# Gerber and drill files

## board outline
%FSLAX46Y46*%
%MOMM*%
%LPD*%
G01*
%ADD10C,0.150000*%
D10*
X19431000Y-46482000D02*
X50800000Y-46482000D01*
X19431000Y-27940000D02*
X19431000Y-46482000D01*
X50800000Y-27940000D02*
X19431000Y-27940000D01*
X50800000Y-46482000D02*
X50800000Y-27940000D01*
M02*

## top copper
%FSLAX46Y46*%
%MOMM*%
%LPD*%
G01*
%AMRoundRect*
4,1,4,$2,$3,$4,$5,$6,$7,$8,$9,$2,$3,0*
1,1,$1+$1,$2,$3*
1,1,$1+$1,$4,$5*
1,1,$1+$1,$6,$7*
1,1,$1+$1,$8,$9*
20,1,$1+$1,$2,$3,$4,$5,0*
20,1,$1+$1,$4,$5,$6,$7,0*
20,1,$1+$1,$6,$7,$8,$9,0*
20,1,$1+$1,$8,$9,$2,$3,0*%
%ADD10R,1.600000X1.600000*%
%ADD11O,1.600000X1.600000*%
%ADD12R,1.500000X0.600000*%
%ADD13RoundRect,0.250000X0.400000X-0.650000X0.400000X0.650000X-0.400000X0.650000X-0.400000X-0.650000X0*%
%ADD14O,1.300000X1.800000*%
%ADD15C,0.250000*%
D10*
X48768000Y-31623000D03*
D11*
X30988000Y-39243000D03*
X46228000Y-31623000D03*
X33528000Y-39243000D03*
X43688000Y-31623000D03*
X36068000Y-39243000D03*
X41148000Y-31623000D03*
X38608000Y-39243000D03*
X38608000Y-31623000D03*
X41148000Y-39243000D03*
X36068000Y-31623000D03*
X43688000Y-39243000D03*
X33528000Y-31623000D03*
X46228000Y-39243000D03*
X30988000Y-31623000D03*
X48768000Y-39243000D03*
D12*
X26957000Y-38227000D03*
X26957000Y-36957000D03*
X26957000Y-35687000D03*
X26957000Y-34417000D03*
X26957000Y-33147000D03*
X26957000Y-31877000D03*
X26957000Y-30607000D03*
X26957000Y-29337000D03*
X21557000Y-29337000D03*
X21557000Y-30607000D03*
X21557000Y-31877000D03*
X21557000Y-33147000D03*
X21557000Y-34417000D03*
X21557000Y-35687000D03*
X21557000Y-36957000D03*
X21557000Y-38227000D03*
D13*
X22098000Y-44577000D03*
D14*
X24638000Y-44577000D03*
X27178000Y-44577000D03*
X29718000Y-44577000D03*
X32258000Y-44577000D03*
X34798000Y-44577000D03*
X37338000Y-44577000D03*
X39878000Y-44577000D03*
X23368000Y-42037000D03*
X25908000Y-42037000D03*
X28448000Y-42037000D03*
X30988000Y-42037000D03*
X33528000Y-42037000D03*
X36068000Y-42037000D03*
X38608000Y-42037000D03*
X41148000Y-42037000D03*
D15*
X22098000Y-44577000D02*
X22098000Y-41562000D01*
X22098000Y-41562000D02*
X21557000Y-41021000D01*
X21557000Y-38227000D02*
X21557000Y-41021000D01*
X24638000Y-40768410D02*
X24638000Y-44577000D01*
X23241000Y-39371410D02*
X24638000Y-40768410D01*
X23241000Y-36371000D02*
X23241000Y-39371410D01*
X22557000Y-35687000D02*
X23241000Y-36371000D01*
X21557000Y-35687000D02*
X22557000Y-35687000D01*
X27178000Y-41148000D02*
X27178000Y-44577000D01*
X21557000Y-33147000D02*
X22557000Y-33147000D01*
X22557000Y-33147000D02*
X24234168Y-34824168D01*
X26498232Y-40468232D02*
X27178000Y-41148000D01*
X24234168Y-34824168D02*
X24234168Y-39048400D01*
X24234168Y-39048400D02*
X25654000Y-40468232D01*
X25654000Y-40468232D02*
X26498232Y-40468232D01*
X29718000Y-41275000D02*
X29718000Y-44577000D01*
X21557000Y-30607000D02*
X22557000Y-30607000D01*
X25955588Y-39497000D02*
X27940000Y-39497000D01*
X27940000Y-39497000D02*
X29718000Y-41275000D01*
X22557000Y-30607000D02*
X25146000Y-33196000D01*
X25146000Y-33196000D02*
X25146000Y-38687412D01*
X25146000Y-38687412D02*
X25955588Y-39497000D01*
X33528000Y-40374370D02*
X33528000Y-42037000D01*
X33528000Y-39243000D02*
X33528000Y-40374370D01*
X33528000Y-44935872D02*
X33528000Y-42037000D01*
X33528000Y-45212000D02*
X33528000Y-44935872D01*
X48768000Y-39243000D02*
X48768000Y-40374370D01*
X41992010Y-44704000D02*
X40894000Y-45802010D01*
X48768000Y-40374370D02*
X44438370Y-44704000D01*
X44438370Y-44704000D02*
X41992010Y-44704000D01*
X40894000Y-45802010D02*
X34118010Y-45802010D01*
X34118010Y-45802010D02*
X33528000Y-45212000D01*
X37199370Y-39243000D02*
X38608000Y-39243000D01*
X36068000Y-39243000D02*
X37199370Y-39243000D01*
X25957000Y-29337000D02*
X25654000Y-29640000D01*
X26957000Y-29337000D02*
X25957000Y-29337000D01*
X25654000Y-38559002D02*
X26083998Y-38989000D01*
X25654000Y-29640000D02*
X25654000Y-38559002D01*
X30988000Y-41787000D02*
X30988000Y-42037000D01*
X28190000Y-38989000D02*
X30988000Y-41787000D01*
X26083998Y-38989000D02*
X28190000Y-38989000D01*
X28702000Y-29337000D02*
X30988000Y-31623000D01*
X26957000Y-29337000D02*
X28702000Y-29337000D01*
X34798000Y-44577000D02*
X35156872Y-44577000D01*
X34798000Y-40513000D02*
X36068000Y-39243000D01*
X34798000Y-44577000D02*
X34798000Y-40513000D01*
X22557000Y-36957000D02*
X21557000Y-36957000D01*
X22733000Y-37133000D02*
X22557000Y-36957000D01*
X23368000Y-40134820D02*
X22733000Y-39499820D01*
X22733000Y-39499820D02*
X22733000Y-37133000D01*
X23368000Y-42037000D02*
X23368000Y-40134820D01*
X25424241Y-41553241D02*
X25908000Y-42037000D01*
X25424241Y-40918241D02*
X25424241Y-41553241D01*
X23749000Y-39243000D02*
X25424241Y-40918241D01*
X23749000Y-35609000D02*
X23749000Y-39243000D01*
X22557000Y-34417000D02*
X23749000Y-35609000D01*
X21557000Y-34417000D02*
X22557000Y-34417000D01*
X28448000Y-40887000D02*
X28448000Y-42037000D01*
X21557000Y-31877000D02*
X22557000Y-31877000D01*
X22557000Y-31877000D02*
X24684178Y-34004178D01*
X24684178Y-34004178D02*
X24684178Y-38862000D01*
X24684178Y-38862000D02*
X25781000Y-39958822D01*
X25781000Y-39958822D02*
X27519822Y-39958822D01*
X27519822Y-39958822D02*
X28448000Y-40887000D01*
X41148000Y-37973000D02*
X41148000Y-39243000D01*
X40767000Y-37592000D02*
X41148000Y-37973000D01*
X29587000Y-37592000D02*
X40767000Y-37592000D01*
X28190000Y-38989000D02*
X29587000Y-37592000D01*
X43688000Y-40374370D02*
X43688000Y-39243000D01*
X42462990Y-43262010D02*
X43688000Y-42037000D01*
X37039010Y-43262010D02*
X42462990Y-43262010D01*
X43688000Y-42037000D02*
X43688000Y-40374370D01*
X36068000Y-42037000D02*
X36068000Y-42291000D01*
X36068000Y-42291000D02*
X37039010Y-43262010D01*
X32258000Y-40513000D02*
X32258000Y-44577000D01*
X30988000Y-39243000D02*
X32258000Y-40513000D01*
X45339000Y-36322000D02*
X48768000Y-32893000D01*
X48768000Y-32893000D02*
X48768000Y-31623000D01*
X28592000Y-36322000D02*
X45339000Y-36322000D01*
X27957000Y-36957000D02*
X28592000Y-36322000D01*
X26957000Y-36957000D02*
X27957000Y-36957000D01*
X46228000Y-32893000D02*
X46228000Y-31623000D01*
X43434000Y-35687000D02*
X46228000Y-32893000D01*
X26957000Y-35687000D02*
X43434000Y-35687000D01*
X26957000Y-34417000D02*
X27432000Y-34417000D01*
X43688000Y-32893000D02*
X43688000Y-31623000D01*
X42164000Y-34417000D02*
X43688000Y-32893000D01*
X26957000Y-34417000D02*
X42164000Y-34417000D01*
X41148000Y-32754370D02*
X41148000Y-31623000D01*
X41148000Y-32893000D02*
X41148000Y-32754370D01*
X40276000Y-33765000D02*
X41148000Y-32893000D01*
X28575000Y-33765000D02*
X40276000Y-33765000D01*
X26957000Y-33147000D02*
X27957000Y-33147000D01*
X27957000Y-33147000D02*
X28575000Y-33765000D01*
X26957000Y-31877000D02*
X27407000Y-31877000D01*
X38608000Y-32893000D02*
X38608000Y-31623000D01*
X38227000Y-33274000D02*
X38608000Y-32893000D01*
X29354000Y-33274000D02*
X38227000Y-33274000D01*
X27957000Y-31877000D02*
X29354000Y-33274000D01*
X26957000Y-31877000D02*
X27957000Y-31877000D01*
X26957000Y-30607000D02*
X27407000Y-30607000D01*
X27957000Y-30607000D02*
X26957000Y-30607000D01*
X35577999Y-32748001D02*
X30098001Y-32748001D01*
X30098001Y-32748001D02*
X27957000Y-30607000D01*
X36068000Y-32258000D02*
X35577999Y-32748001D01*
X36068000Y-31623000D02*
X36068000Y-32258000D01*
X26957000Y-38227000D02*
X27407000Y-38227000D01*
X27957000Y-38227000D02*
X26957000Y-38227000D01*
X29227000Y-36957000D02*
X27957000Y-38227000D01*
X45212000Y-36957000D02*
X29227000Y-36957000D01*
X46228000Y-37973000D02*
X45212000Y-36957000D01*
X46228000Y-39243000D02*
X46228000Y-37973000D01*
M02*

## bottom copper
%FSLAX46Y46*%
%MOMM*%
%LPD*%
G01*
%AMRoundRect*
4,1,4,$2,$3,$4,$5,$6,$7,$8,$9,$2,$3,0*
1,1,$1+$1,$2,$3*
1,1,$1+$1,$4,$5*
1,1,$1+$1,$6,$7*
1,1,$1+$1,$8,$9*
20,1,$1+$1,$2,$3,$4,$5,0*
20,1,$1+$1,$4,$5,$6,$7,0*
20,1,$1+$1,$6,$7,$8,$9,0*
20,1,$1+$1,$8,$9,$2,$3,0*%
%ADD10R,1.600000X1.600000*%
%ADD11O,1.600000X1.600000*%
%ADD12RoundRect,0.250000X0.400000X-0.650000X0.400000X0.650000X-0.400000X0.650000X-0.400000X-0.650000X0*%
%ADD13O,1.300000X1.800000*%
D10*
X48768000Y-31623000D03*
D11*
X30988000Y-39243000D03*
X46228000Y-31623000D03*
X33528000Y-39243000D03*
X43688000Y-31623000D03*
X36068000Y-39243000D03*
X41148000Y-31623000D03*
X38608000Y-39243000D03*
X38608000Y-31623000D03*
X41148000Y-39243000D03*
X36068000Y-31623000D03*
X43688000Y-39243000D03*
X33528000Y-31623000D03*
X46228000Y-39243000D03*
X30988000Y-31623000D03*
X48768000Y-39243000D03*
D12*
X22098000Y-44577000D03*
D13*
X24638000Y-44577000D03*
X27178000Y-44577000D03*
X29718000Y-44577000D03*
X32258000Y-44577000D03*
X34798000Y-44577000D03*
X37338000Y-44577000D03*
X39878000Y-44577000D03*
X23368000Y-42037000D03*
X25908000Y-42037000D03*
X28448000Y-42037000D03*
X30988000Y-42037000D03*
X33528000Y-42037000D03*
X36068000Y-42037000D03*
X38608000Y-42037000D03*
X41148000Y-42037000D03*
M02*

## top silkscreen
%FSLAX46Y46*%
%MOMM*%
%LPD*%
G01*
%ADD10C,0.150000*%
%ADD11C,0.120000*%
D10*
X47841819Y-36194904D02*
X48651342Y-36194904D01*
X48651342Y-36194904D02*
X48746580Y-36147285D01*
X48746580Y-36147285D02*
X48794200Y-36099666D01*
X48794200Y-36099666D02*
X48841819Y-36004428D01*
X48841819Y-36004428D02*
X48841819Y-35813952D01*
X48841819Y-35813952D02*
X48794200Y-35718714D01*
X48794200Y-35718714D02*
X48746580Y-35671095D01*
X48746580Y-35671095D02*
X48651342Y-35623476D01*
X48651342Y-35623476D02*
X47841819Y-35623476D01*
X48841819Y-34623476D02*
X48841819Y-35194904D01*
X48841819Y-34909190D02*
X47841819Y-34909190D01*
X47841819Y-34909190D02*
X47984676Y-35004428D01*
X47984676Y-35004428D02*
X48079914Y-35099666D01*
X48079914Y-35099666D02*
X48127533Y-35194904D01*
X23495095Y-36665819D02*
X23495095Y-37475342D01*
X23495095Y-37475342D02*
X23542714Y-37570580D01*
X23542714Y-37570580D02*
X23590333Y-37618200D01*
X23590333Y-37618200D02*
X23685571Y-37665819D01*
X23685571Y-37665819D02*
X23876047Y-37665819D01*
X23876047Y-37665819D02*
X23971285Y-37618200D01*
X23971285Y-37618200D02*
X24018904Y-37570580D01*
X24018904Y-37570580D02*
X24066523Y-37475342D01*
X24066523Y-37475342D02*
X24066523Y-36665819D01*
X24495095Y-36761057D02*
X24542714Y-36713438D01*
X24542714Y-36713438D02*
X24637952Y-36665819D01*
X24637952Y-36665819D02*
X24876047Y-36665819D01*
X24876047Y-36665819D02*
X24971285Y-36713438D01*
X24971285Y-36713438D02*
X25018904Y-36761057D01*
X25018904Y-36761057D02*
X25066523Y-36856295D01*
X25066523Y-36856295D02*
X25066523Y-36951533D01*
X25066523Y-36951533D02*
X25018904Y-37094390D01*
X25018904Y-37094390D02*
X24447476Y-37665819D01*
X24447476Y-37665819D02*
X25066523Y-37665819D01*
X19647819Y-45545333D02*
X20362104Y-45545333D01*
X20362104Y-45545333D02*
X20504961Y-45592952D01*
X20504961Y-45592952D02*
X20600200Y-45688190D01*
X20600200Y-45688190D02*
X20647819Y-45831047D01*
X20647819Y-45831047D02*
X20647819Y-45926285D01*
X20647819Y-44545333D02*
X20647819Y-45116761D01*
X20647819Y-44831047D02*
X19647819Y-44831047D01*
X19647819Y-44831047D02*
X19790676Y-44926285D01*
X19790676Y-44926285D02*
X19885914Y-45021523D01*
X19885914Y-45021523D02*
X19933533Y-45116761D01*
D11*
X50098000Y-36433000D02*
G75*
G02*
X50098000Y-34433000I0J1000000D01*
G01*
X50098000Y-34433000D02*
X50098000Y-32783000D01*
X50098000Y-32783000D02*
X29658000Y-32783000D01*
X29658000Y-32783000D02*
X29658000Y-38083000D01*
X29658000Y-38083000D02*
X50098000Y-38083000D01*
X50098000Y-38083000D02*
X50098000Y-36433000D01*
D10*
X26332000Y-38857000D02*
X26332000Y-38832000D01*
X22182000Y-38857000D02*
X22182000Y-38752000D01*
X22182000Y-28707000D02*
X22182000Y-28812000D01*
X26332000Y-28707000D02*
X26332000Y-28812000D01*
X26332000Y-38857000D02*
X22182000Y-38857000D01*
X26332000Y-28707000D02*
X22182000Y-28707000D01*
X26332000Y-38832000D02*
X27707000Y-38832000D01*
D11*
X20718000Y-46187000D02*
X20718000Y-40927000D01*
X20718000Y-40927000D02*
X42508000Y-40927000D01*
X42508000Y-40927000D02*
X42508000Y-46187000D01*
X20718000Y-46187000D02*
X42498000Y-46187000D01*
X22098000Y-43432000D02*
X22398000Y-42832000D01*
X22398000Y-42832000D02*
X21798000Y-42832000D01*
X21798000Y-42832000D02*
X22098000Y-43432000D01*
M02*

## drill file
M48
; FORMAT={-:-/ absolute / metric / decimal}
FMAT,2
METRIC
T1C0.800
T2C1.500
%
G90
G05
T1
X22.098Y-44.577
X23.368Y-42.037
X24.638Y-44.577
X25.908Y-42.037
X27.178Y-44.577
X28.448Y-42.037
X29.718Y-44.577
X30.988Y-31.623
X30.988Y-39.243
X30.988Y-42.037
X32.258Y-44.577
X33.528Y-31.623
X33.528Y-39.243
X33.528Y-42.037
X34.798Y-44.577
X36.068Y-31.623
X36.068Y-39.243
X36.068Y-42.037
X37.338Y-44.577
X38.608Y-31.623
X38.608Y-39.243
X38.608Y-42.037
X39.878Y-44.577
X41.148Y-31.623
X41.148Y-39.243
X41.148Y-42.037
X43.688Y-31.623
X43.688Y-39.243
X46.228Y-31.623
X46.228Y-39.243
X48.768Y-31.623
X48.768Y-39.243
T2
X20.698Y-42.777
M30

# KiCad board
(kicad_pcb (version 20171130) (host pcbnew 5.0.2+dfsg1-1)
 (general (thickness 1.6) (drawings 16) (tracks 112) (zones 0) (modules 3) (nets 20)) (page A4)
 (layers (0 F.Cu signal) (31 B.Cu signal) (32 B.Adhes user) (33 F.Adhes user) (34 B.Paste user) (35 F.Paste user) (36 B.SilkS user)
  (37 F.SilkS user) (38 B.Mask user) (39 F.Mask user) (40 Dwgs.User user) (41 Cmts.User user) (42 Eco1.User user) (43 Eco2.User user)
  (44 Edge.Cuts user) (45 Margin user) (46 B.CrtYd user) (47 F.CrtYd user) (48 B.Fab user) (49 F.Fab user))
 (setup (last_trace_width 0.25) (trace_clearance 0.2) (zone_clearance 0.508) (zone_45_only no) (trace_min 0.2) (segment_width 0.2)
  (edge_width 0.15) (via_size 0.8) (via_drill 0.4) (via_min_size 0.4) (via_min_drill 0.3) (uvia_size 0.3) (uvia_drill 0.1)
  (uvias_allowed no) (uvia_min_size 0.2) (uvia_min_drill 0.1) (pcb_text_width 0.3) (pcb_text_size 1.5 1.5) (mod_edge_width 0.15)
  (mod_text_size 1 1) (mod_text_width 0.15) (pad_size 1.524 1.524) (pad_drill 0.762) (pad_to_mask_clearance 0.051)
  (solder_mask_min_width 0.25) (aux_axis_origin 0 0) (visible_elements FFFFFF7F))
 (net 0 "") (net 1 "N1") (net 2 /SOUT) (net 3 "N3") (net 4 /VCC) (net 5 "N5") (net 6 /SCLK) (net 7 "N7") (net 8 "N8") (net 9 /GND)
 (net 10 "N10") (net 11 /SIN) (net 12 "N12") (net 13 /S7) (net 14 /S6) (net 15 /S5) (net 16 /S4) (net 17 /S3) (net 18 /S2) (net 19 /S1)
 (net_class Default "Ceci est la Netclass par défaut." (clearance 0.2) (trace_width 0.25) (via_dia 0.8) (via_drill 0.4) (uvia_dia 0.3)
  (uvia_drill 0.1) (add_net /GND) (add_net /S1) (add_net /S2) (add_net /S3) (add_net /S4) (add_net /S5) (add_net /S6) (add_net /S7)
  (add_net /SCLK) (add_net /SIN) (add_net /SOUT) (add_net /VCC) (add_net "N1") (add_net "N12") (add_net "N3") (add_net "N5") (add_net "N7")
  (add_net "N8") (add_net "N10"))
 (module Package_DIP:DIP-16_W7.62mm (layer F.Cu) (at 48.768 31.623 270)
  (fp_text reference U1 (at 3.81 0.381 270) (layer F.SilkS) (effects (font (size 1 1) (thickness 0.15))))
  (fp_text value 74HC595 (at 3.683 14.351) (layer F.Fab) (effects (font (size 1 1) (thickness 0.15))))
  (fp_arc (start 3.81 -1.33) (end 2.81 -1.33) (angle -180) (layer F.SilkS) (width 0.12))
  (fp_line (start 2.81 -1.33) (end 1.16 -1.33) (layer F.SilkS) (width 0.12))
  (fp_line (start 1.16 -1.33) (end 1.16 19.11) (layer F.SilkS) (width 0.12))
  (fp_line (start 1.16 19.11) (end 6.46 19.11) (layer F.SilkS) (width 0.12))
  (fp_line (start 6.46 19.11) (end 6.46 -1.33) (layer F.SilkS) (width 0.12))
  (fp_line (start 6.46 -1.33) (end 4.81 -1.33) (layer F.SilkS) (width 0.12))
  (pad 1 thru_hole rect (at 0 0 270) (size 1.6 1.6) (drill 0.8) (layers *.Cu *.Mask) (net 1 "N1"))
  (pad 9 thru_hole oval (at 7.62 17.78 270) (size 1.6 1.6) (drill 0.8) (layers *.Cu *.Mask) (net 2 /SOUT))
  (pad 2 thru_hole oval (at 0 2.54 270) (size 1.6 1.6) (drill 0.8) (layers *.Cu *.Mask) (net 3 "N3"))
  (pad 10 thru_hole oval (at 7.62 15.24 270) (size 1.6 1.6) (drill 0.8) (layers *.Cu *.Mask) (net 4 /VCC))
  (pad 3 thru_hole oval (at 0 5.08 270) (size 1.6 1.6) (drill 0.8) (layers *.Cu *.Mask) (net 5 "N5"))
  (pad 11 thru_hole oval (at 7.62 12.7 270) (size 1.6 1.6) (drill 0.8) (layers *.Cu *.Mask) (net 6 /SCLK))
  (pad 4 thru_hole oval (at 0 7.62 270) (size 1.6 1.6) (drill 0.8) (layers *.Cu *.Mask) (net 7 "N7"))
  (pad 12 thru_hole oval (at 7.62 10.16 270) (size 1.6 1.6) (drill 0.8) (layers *.Cu *.Mask) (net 6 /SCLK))
  (pad 5 thru_hole oval (at 0 10.16 270) (size 1.6 1.6) (drill 0.8) (layers *.Cu *.Mask) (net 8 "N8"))
  (pad 13 thru_hole oval (at 7.62 7.62 270) (size 1.6 1.6) (drill 0.8) (layers *.Cu *.Mask) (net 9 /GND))
  (pad 6 thru_hole oval (at 0 12.7 270) (size 1.6 1.6) (drill 0.8) (layers *.Cu *.Mask) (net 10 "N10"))
  (pad 14 thru_hole oval (at 7.62 5.08 270) (size 1.6 1.6) (drill 0.8) (layers *.Cu *.Mask) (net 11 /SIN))
  (pad 7 thru_hole oval (at 0 15.24 270) (size 1.6 1.6) (drill 0.8) (layers *.Cu *.Mask))
  (pad 15 thru_hole oval (at 7.62 2.54 270) (size 1.6 1.6) (drill 0.8) (layers *.Cu *.Mask) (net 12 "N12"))
  (pad 8 thru_hole oval (at 0 17.78 270) (size 1.6 1.6) (drill 0.8) (layers *.Cu *.Mask) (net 9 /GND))
  (pad 16 thru_hole oval (at 7.62 0 270) (size 1.6 1.6) (drill 0.8) (layers *.Cu *.Mask) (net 4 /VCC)))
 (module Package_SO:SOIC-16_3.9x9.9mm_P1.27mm (layer F.Cu) (at 24.257 33.782 180)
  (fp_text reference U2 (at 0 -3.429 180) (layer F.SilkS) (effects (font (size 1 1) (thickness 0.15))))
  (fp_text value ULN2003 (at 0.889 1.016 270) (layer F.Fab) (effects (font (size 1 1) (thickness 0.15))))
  (fp_line (start -2.075 -5.075) (end -2.075 -5.05) (layer F.SilkS) (width 0.15))
  (fp_line (start 2.075 -5.075) (end 2.075 -4.97) (layer F.SilkS) (width 0.15))
  (fp_line (start 2.075 5.075) (end 2.075 4.97) (layer F.SilkS) (width 0.15))
  (fp_line (start -2.075 5.075) (end -2.075 4.97) (layer F.SilkS) (width 0.15))
  (fp_line (start -2.075 -5.075) (end 2.075 -5.075) (layer F.SilkS) (width 0.15))
  (fp_line (start -2.075 5.075) (end 2.075 5.075) (layer F.SilkS) (width 0.15))
  (fp_line (start -2.075 -5.05) (end -3.45 -5.05) (layer F.SilkS) (width 0.15))
  (pad 1 smd rect (at -2.7 -4.445 180) (size 1.5 0.6) (layers F.Cu F.Paste F.Mask) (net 12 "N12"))
  (pad 2 smd rect (at -2.7 -3.175 180) (size 1.5 0.6) (layers F.Cu F.Paste F.Mask) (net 1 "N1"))
  (pad 3 smd rect (at -2.7 -1.905 180) (size 1.5 0.6) (layers F.Cu F.Paste F.Mask) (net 3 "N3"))
  (pad 4 smd rect (at -2.7 -0.635 180) (size 1.5 0.6) (layers F.Cu F.Paste F.Mask) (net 5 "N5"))
  (pad 5 smd rect (at -2.7 0.635 180) (size 1.5 0.6) (layers F.Cu F.Paste F.Mask) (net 7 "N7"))
  (pad 6 smd rect (at -2.7 1.905 180) (size 1.5 0.6) (layers F.Cu F.Paste F.Mask) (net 8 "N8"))
  (pad 7 smd rect (at -2.7 3.175 180) (size 1.5 0.6) (layers F.Cu F.Paste F.Mask) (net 10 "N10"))
  (pad 8 smd rect (at -2.7 4.445 180) (size 1.5 0.6) (layers F.Cu F.Paste F.Mask) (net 9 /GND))
  (pad 9 smd rect (at 2.7 4.445 180) (size 1.5 0.6) (layers F.Cu F.Paste F.Mask))
  (pad 10 smd rect (at 2.7 3.175 180) (size 1.5 0.6) (layers F.Cu F.Paste F.Mask) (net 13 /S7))
  (pad 11 smd rect (at 2.7 1.905 180) (size 1.5 0.6) (layers F.Cu F.Paste F.Mask) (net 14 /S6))
  (pad 12 smd rect (at 2.7 0.635 180) (size 1.5 0.6) (layers F.Cu F.Paste F.Mask) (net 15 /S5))
  (pad 13 smd rect (at 2.7 -0.635 180) (size 1.5 0.6) (layers F.Cu F.Paste F.Mask) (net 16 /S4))
  (pad 14 smd rect (at 2.7 -1.905 180) (size 1.5 0.6) (layers F.Cu F.Paste F.Mask) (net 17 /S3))
  (pad 15 smd rect (at 2.7 -3.175 180) (size 1.5 0.6) (layers F.Cu F.Paste F.Mask) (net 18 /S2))
  (pad 16 smd rect (at 2.7 -4.445 180) (size 1.5 0.6) (layers F.Cu F.Paste F.Mask) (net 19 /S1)))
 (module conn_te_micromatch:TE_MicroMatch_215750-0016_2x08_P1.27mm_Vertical (layer F.Cu) (at 22.098 44.577 90)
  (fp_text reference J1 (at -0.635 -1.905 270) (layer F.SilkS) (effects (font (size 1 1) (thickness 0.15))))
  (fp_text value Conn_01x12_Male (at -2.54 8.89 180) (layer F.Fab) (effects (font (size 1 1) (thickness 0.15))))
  (fp_line (start -1.61 -1.38) (end 3.65 -1.38) (layer F.SilkS) (width 0.12))
  (fp_line (start 3.65 -1.38) (end 3.65 20.41) (layer F.SilkS) (width 0.12))
  (fp_line (start 3.65 20.41) (end -1.61 20.41) (layer F.SilkS) (width 0.12))
  (fp_line (start -1.61 -1.38) (end -1.61 20.4) (layer F.SilkS) (width 0.12))
  (fp_line (start 1.145 0) (end 1.745 0.3) (layer F.SilkS) (width 0.12))
  (fp_line (start 1.745 0.3) (end 1.745 -0.3) (layer F.SilkS) (width 0.12))
  (fp_line (start 1.745 -0.3) (end 1.145 0) (layer F.SilkS) (width 0.12))
  (pad 1 thru_hole roundrect (at 0 0 90) (size 1.8 1.3) (drill 0.8) (layers *.Cu *.Mask) (roundrect_rratio 0.192308) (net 19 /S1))
  (pad 3 thru_hole oval (at 0 2.54 90) (size 1.8 1.3) (drill 0.8) (layers *.Cu *.Mask) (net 17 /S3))
  (pad 5 thru_hole oval (at 0 5.08 90) (size 1.8 1.3) (drill 0.8) (layers *.Cu *.Mask) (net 15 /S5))
  (pad 7 thru_hole oval (at 0 7.62 90) (size 1.8 1.3) (drill 0.8) (layers *.Cu *.Mask) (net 13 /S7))
  (pad 9 thru_hole oval (at 0 10.16 90) (size 1.8 1.3) (drill 0.8) (layers *.Cu *.Mask) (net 2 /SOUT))
  (pad 11 thru_hole oval (at 0 12.7 90) (size 1.8 1.3) (drill 0.8) (layers *.Cu *.Mask) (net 6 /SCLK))
  (pad 13 thru_hole oval (at 0 15.24 90) (size 1.8 1.3) (drill 0.8) (layers *.Cu *.Mask))
  (pad 15 thru_hole oval (at 0 17.78 90) (size 1.8 1.3) (drill 0.8) (layers *.Cu *.Mask))
  (pad 2 thru_hole oval (at 2.54 1.27 90) (size 1.8 1.3) (drill 0.8) (layers *.Cu *.Mask) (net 18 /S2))
  (pad 4 thru_hole oval (at 2.54 3.81 90) (size 1.8 1.3) (drill 0.8) (layers *.Cu *.Mask) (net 16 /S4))
  (pad 6 thru_hole oval (at 2.54 6.35 90) (size 1.8 1.3) (drill 0.8) (layers *.Cu *.Mask) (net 14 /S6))
  (pad 8 thru_hole oval (at 2.54 8.89 90) (size 1.8 1.3) (drill 0.8) (layers *.Cu *.Mask) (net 9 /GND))
  (pad 10 thru_hole oval (at 2.54 11.43 90) (size 1.8 1.3) (drill 0.8) (layers *.Cu *.Mask) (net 4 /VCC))
  (pad 12 thru_hole oval (at 2.54 13.97 90) (size 1.8 1.3) (drill 0.8) (layers *.Cu *.Mask) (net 11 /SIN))
  (pad 14 thru_hole oval (at 2.54 16.51 90) (size 1.8 1.3) (drill 0.8) (layers *.Cu *.Mask))
  (pad 16 thru_hole oval (at 2.54 19.05 90) (size 1.8 1.3) (drill 0.8) (layers *.Cu *.Mask))
  (pad "" np_thru_hole circle (at 1.8 -1.4 90) (size 1.5 1.5) (drill 1.5) (layers *.Cu *.Mask)))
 (gr_line (start 19.431 46.482) (end 50.8 46.482) (layer Edge.Cuts) (width 0.15))
 (gr_line (start 19.431 27.94) (end 19.431 46.482) (layer Edge.Cuts) (width 0.15))
 (gr_line (start 50.8 27.94) (end 19.431 27.94) (layer Edge.Cuts) (width 0.15))
 (gr_line (start 50.8 46.482) (end 50.8 27.94) (layer Edge.Cuts) (width 0.15))
 (segment (start 22.098 44.577) (end 22.098 41.562) (width 0.25) (layer F.Cu) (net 19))
 (segment (start 22.098 41.562) (end 21.557 41.021) (width 0.25) (layer F.Cu) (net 19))
 (segment (start 21.557 38.227) (end 21.557 41.021) (width 0.25) (layer F.Cu) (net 19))
 (segment (start 24.638 40.76841) (end 24.638 44.577) (width 0.25) (layer F.Cu) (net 17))
 (segment (start 23.241 39.37141) (end 24.638 40.76841) (width 0.25) (layer F.Cu) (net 17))
 (segment (start 23.241 36.371) (end 23.241 39.37141) (width 0.25) (layer F.Cu) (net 17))
 (segment (start 22.557 35.687) (end 23.241 36.371) (width 0.25) (layer F.Cu) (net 17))
 (segment (start 21.557 35.687) (end 22.557 35.687) (width 0.25) (layer F.Cu) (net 17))
 (segment (start 27.178 41.148) (end 27.178 44.577) (width 0.25) (layer F.Cu) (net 15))
 (segment (start 21.557 33.147) (end 22.557 33.147) (width 0.25) (layer F.Cu) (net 15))
 (segment (start 22.557 33.147) (end 24.234168 34.824168) (width 0.25) (layer F.Cu) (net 15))
 (segment (start 26.498232 40.468232) (end 27.178 41.148) (width 0.25) (layer F.Cu) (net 15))
 (segment (start 24.234168 34.824168) (end 24.234168 39.0484) (width 0.25) (layer F.Cu) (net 15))
 (segment (start 24.234168 39.0484) (end 25.654 40.468232) (width 0.25) (layer F.Cu) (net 15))
 (segment (start 25.654 40.468232) (end 26.498232 40.468232) (width 0.25) (layer F.Cu) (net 15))
 (segment (start 29.718 41.275) (end 29.718 44.577) (width 0.25) (layer F.Cu) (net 13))
 (segment (start 21.557 30.607) (end 22.557 30.607) (width 0.25) (layer F.Cu) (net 13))
 (segment (start 25.955588 39.497) (end 27.94 39.497) (width 0.25) (layer F.Cu) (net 13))
 (segment (start 27.94 39.497) (end 29.718 41.275) (width 0.25) (layer F.Cu) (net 13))
 (segment (start 22.557 30.607) (end 25.146 33.196) (width 0.25) (layer F.Cu) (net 13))
 (segment (start 25.146 33.196) (end 25.146 38.687412) (width 0.25) (layer F.Cu) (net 13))
 (segment (start 25.146 38.687412) (end 25.955588 39.497) (width 0.25) (layer F.Cu) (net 13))
 (segment (start 33.528 40.37437) (end 33.528 42.037) (width 0.25) (layer F.Cu) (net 4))
 (segment (start 33.528 39.243) (end 33.528 40.37437) (width 0.25) (layer F.Cu) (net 4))
 (segment (start 33.528 44.935872) (end 33.528 42.037) (width 0.25) (layer F.Cu) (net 4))
 (segment (start 33.528 45.212) (end 33.528 44.935872) (width 0.25) (layer F.Cu) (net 4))
 (segment (start 48.768 39.243) (end 48.768 40.37437) (width 0.25) (layer F.Cu) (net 4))
 (segment (start 41.99201 44.704) (end 40.894 45.80201) (width 0.25) (layer F.Cu) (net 4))
 (segment (start 48.768 40.37437) (end 44.43837 44.704) (width 0.25) (layer F.Cu) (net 4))
 (segment (start 44.43837 44.704) (end 41.99201 44.704) (width 0.25) (layer F.Cu) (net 4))
 (segment (start 40.894 45.80201) (end 34.11801 45.80201) (width 0.25) (layer F.Cu) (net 4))
 (segment (start 34.11801 45.80201) (end 33.528 45.212) (width 0.25) (layer F.Cu) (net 4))
 (segment (start 37.19937 39.243) (end 38.608 39.243) (width 0.25) (layer F.Cu) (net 6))
 (segment (start 36.068 39.243) (end 37.19937 39.243) (width 0.25) (layer F.Cu) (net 6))
 (segment (start 25.957 29.337) (end 25.654 29.64) (width 0.25) (layer F.Cu) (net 9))
 (segment (start 26.957 29.337) (end 25.957 29.337) (width 0.25) (layer F.Cu) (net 9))
 (segment (start 25.654 38.559002) (end 26.083998 38.989) (width 0.25) (layer F.Cu) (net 9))
 (segment (start 25.654 29.64) (end 25.654 38.559002) (width 0.25) (layer F.Cu) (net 9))
 (segment (start 30.988 41.787) (end 30.988 42.037) (width 0.25) (layer F.Cu) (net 9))
 (segment (start 28.19 38.989) (end 30.988 41.787) (width 0.25) (layer F.Cu) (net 9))
 (segment (start 26.083998 38.989) (end 28.19 38.989) (width 0.25) (layer F.Cu) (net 9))
 (segment (start 28.702 29.337) (end 30.988 31.623) (width 0.25) (layer F.Cu) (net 9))
 (segment (start 26.957 29.337) (end 28.702 29.337) (width 0.25) (layer F.Cu) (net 9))
 (segment (start 34.798 44.577) (end 35.156872 44.577) (width 0.25) (layer F.Cu) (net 6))
 (segment (start 34.798 40.513) (end 36.068 39.243) (width 0.25) (layer F.Cu) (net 6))
 (segment (start 34.798 44.577) (end 34.798 40.513) (width 0.25) (layer F.Cu) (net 6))
 (segment (start 22.557 36.957) (end 21.557 36.957) (width 0.25) (layer F.Cu) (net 18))
 (segment (start 22.733 37.133) (end 22.557 36.957) (width 0.25) (layer F.Cu) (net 18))
 (segment (start 23.368 40.13482) (end 22.733 39.49982) (width 0.25) (layer F.Cu) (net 18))
 (segment (start 22.733 39.49982) (end 22.733 37.133) (width 0.25) (layer F.Cu) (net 18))
 (segment (start 23.368 42.037) (end 23.368 40.13482) (width 0.25) (layer F.Cu) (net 18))
 (segment (start 25.424241 41.553241) (end 25.908 42.037) (width 0.25) (layer F.Cu) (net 16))
 (segment (start 25.424241 40.918241) (end 25.424241 41.553241) (width 0.25) (layer F.Cu) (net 16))
 (segment (start 23.749 39.243) (end 25.424241 40.918241) (width 0.25) (layer F.Cu) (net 16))
 (segment (start 23.749 35.609) (end 23.749 39.243) (width 0.25) (layer F.Cu) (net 16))
 (segment (start 22.557 34.417) (end 23.749 35.609) (width 0.25) (layer F.Cu) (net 16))
 (segment (start 21.557 34.417) (end 22.557 34.417) (width 0.25) (layer F.Cu) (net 16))
 (segment (start 28.448 40.887) (end 28.448 42.037) (width 0.25) (layer F.Cu) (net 14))
 (segment (start 21.557 31.877) (end 22.557 31.877) (width 0.25) (layer F.Cu) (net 14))
 (segment (start 22.557 31.877) (end 24.684178 34.004178) (width 0.25) (layer F.Cu) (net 14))
 (segment (start 24.684178 34.004178) (end 24.684178 38.862) (width 0.25) (layer F.Cu) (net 14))
 (segment (start 24.684178 38.862) (end 25.781 39.958822) (width 0.25) (layer F.Cu) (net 14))
 (segment (start 25.781 39.958822) (end 27.519822 39.958822) (width 0.25) (layer F.Cu) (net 14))
 (segment (start 27.519822 39.958822) (end 28.448 40.887) (width 0.25) (layer F.Cu) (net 14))
 (segment (start 41.148 37.973) (end 41.148 39.243) (width 0.25) (layer F.Cu) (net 9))
 (segment (start 40.767 37.592) (end 41.148 37.973) (width 0.25) (layer F.Cu) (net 9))
 (segment (start 29.587 37.592) (end 40.767 37.592) (width 0.25) (layer F.Cu) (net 9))
 (segment (start 28.19 38.989) (end 29.587 37.592) (width 0.25) (layer F.Cu) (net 9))
 (segment (start 43.688 40.37437) (end 43.688 39.243) (width 0.25) (layer F.Cu) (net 11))
 (segment (start 42.46299 43.26201) (end 43.688 42.037) (width 0.25) (layer F.Cu) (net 11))
 (segment (start 37.03901 43.26201) (end 42.46299 43.26201) (width 0.25) (layer F.Cu) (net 11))
 (segment (start 43.688 42.037) (end 43.688 40.37437) (width 0.25) (layer F.Cu) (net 11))
 (segment (start 36.068 42.037) (end 36.068 42.291) (width 0.25) (layer F.Cu) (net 11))
 (segment (start 36.068 42.291) (end 37.03901 43.26201) (width 0.25) (layer F.Cu) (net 11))
 (segment (start 32.258 40.513) (end 32.258 44.577) (width 0.25) (layer F.Cu) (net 2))
 (segment (start 30.988 39.243) (end 32.258 40.513) (width 0.25) (layer F.Cu) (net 2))
 (segment (start 45.339 36.322) (end 48.768 32.893) (width 0.25) (layer F.Cu) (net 1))
 (segment (start 48.768 32.893) (end 48.768 31.623) (width 0.25) (layer F.Cu) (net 1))
 (segment (start 28.592 36.322) (end 45.339 36.322) (width 0.25) (layer F.Cu) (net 1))
 (segment (start 27.957 36.957) (end 28.592 36.322) (width 0.25) (layer F.Cu) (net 1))
 (segment (start 26.957 36.957) (end 27.957 36.957) (width 0.25) (layer F.Cu) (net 1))
 (segment (start 46.228 32.893) (end 46.228 31.623) (width 0.25) (layer F.Cu) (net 3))
 (segment (start 43.434 35.687) (end 46.228 32.893) (width 0.25) (layer F.Cu) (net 3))
 (segment (start 26.957 35.687) (end 43.434 35.687) (width 0.25) (layer F.Cu) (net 3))
 (segment (start 26.957 34.417) (end 27.432 34.417) (width 0.25) (layer F.Cu) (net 5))
 (segment (start 43.688 32.893) (end 43.688 31.623) (width 0.25) (layer F.Cu) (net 5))
 (segment (start 42.164 34.417) (end 43.688 32.893) (width 0.25) (layer F.Cu) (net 5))
 (segment (start 26.957 34.417) (end 42.164 34.417) (width 0.25) (layer F.Cu) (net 5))
 (segment (start 41.148 32.75437) (end 41.148 31.623) (width 0.25) (layer F.Cu) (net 7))
 (segment (start 41.148 32.893) (end 41.148 32.75437) (width 0.25) (layer F.Cu) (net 7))
 (segment (start 40.276 33.765) (end 41.148 32.893) (width 0.25) (layer F.Cu) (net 7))
 (segment (start 28.575 33.765) (end 40.276 33.765) (width 0.25) (layer F.Cu) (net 7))
 (segment (start 26.957 33.147) (end 27.957 33.147) (width 0.25) (layer F.Cu) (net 7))
 (segment (start 27.957 33.147) (end 28.575 33.765) (width 0.25) (layer F.Cu) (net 7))
 (segment (start 26.957 31.877) (end 27.407 31.877) (width 0.25) (layer F.Cu) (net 8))
 (segment (start 38.608 32.893) (end 38.608 31.623) (width 0.25) (layer F.Cu) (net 8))
 (segment (start 38.227 33.274) (end 38.608 32.893) (width 0.25) (layer F.Cu) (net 8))
 (segment (start 29.354 33.274) (end 38.227 33.274) (width 0.25) (layer F.Cu) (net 8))
 (segment (start 27.957 31.877) (end 29.354 33.274) (width 0.25) (layer F.Cu) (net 8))
 (segment (start 26.957 31.877) (end 27.957 31.877) (width 0.25) (layer F.Cu) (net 8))
 (segment (start 26.957 30.607) (end 27.407 30.607) (width 0.25) (layer F.Cu) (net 10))
 (segment (start 27.957 30.607) (end 26.957 30.607) (width 0.25) (layer F.Cu) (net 10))
 (segment (start 35.577999 32.748001) (end 30.098001 32.748001) (width 0.25) (layer F.Cu) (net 10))
 (segment (start 30.098001 32.748001) (end 27.957 30.607) (width 0.25) (layer F.Cu) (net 10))
 (segment (start 36.068 32.258) (end 35.577999 32.748001) (width 0.25) (layer F.Cu) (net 10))
 (segment (start 36.068 31.623) (end 36.068 32.258) (width 0.25) (layer F.Cu) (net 10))
 (segment (start 26.957 38.227) (end 27.407 38.227) (width 0.25) (layer F.Cu) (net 12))
 (segment (start 27.957 38.227) (end 26.957 38.227) (width 0.25) (layer F.Cu) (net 12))
 (segment (start 29.227 36.957) (end 27.957 38.227) (width 0.25) (layer F.Cu) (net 12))
 (segment (start 45.212 36.957) (end 29.227 36.957) (width 0.25) (layer F.Cu) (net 12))
 (segment (start 46.228 37.973) (end 45.212 36.957) (width 0.25) (layer F.Cu) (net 12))
 (segment (start 46.228 39.243) (end 46.228 37.973) (width 0.25) (layer F.Cu) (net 12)))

